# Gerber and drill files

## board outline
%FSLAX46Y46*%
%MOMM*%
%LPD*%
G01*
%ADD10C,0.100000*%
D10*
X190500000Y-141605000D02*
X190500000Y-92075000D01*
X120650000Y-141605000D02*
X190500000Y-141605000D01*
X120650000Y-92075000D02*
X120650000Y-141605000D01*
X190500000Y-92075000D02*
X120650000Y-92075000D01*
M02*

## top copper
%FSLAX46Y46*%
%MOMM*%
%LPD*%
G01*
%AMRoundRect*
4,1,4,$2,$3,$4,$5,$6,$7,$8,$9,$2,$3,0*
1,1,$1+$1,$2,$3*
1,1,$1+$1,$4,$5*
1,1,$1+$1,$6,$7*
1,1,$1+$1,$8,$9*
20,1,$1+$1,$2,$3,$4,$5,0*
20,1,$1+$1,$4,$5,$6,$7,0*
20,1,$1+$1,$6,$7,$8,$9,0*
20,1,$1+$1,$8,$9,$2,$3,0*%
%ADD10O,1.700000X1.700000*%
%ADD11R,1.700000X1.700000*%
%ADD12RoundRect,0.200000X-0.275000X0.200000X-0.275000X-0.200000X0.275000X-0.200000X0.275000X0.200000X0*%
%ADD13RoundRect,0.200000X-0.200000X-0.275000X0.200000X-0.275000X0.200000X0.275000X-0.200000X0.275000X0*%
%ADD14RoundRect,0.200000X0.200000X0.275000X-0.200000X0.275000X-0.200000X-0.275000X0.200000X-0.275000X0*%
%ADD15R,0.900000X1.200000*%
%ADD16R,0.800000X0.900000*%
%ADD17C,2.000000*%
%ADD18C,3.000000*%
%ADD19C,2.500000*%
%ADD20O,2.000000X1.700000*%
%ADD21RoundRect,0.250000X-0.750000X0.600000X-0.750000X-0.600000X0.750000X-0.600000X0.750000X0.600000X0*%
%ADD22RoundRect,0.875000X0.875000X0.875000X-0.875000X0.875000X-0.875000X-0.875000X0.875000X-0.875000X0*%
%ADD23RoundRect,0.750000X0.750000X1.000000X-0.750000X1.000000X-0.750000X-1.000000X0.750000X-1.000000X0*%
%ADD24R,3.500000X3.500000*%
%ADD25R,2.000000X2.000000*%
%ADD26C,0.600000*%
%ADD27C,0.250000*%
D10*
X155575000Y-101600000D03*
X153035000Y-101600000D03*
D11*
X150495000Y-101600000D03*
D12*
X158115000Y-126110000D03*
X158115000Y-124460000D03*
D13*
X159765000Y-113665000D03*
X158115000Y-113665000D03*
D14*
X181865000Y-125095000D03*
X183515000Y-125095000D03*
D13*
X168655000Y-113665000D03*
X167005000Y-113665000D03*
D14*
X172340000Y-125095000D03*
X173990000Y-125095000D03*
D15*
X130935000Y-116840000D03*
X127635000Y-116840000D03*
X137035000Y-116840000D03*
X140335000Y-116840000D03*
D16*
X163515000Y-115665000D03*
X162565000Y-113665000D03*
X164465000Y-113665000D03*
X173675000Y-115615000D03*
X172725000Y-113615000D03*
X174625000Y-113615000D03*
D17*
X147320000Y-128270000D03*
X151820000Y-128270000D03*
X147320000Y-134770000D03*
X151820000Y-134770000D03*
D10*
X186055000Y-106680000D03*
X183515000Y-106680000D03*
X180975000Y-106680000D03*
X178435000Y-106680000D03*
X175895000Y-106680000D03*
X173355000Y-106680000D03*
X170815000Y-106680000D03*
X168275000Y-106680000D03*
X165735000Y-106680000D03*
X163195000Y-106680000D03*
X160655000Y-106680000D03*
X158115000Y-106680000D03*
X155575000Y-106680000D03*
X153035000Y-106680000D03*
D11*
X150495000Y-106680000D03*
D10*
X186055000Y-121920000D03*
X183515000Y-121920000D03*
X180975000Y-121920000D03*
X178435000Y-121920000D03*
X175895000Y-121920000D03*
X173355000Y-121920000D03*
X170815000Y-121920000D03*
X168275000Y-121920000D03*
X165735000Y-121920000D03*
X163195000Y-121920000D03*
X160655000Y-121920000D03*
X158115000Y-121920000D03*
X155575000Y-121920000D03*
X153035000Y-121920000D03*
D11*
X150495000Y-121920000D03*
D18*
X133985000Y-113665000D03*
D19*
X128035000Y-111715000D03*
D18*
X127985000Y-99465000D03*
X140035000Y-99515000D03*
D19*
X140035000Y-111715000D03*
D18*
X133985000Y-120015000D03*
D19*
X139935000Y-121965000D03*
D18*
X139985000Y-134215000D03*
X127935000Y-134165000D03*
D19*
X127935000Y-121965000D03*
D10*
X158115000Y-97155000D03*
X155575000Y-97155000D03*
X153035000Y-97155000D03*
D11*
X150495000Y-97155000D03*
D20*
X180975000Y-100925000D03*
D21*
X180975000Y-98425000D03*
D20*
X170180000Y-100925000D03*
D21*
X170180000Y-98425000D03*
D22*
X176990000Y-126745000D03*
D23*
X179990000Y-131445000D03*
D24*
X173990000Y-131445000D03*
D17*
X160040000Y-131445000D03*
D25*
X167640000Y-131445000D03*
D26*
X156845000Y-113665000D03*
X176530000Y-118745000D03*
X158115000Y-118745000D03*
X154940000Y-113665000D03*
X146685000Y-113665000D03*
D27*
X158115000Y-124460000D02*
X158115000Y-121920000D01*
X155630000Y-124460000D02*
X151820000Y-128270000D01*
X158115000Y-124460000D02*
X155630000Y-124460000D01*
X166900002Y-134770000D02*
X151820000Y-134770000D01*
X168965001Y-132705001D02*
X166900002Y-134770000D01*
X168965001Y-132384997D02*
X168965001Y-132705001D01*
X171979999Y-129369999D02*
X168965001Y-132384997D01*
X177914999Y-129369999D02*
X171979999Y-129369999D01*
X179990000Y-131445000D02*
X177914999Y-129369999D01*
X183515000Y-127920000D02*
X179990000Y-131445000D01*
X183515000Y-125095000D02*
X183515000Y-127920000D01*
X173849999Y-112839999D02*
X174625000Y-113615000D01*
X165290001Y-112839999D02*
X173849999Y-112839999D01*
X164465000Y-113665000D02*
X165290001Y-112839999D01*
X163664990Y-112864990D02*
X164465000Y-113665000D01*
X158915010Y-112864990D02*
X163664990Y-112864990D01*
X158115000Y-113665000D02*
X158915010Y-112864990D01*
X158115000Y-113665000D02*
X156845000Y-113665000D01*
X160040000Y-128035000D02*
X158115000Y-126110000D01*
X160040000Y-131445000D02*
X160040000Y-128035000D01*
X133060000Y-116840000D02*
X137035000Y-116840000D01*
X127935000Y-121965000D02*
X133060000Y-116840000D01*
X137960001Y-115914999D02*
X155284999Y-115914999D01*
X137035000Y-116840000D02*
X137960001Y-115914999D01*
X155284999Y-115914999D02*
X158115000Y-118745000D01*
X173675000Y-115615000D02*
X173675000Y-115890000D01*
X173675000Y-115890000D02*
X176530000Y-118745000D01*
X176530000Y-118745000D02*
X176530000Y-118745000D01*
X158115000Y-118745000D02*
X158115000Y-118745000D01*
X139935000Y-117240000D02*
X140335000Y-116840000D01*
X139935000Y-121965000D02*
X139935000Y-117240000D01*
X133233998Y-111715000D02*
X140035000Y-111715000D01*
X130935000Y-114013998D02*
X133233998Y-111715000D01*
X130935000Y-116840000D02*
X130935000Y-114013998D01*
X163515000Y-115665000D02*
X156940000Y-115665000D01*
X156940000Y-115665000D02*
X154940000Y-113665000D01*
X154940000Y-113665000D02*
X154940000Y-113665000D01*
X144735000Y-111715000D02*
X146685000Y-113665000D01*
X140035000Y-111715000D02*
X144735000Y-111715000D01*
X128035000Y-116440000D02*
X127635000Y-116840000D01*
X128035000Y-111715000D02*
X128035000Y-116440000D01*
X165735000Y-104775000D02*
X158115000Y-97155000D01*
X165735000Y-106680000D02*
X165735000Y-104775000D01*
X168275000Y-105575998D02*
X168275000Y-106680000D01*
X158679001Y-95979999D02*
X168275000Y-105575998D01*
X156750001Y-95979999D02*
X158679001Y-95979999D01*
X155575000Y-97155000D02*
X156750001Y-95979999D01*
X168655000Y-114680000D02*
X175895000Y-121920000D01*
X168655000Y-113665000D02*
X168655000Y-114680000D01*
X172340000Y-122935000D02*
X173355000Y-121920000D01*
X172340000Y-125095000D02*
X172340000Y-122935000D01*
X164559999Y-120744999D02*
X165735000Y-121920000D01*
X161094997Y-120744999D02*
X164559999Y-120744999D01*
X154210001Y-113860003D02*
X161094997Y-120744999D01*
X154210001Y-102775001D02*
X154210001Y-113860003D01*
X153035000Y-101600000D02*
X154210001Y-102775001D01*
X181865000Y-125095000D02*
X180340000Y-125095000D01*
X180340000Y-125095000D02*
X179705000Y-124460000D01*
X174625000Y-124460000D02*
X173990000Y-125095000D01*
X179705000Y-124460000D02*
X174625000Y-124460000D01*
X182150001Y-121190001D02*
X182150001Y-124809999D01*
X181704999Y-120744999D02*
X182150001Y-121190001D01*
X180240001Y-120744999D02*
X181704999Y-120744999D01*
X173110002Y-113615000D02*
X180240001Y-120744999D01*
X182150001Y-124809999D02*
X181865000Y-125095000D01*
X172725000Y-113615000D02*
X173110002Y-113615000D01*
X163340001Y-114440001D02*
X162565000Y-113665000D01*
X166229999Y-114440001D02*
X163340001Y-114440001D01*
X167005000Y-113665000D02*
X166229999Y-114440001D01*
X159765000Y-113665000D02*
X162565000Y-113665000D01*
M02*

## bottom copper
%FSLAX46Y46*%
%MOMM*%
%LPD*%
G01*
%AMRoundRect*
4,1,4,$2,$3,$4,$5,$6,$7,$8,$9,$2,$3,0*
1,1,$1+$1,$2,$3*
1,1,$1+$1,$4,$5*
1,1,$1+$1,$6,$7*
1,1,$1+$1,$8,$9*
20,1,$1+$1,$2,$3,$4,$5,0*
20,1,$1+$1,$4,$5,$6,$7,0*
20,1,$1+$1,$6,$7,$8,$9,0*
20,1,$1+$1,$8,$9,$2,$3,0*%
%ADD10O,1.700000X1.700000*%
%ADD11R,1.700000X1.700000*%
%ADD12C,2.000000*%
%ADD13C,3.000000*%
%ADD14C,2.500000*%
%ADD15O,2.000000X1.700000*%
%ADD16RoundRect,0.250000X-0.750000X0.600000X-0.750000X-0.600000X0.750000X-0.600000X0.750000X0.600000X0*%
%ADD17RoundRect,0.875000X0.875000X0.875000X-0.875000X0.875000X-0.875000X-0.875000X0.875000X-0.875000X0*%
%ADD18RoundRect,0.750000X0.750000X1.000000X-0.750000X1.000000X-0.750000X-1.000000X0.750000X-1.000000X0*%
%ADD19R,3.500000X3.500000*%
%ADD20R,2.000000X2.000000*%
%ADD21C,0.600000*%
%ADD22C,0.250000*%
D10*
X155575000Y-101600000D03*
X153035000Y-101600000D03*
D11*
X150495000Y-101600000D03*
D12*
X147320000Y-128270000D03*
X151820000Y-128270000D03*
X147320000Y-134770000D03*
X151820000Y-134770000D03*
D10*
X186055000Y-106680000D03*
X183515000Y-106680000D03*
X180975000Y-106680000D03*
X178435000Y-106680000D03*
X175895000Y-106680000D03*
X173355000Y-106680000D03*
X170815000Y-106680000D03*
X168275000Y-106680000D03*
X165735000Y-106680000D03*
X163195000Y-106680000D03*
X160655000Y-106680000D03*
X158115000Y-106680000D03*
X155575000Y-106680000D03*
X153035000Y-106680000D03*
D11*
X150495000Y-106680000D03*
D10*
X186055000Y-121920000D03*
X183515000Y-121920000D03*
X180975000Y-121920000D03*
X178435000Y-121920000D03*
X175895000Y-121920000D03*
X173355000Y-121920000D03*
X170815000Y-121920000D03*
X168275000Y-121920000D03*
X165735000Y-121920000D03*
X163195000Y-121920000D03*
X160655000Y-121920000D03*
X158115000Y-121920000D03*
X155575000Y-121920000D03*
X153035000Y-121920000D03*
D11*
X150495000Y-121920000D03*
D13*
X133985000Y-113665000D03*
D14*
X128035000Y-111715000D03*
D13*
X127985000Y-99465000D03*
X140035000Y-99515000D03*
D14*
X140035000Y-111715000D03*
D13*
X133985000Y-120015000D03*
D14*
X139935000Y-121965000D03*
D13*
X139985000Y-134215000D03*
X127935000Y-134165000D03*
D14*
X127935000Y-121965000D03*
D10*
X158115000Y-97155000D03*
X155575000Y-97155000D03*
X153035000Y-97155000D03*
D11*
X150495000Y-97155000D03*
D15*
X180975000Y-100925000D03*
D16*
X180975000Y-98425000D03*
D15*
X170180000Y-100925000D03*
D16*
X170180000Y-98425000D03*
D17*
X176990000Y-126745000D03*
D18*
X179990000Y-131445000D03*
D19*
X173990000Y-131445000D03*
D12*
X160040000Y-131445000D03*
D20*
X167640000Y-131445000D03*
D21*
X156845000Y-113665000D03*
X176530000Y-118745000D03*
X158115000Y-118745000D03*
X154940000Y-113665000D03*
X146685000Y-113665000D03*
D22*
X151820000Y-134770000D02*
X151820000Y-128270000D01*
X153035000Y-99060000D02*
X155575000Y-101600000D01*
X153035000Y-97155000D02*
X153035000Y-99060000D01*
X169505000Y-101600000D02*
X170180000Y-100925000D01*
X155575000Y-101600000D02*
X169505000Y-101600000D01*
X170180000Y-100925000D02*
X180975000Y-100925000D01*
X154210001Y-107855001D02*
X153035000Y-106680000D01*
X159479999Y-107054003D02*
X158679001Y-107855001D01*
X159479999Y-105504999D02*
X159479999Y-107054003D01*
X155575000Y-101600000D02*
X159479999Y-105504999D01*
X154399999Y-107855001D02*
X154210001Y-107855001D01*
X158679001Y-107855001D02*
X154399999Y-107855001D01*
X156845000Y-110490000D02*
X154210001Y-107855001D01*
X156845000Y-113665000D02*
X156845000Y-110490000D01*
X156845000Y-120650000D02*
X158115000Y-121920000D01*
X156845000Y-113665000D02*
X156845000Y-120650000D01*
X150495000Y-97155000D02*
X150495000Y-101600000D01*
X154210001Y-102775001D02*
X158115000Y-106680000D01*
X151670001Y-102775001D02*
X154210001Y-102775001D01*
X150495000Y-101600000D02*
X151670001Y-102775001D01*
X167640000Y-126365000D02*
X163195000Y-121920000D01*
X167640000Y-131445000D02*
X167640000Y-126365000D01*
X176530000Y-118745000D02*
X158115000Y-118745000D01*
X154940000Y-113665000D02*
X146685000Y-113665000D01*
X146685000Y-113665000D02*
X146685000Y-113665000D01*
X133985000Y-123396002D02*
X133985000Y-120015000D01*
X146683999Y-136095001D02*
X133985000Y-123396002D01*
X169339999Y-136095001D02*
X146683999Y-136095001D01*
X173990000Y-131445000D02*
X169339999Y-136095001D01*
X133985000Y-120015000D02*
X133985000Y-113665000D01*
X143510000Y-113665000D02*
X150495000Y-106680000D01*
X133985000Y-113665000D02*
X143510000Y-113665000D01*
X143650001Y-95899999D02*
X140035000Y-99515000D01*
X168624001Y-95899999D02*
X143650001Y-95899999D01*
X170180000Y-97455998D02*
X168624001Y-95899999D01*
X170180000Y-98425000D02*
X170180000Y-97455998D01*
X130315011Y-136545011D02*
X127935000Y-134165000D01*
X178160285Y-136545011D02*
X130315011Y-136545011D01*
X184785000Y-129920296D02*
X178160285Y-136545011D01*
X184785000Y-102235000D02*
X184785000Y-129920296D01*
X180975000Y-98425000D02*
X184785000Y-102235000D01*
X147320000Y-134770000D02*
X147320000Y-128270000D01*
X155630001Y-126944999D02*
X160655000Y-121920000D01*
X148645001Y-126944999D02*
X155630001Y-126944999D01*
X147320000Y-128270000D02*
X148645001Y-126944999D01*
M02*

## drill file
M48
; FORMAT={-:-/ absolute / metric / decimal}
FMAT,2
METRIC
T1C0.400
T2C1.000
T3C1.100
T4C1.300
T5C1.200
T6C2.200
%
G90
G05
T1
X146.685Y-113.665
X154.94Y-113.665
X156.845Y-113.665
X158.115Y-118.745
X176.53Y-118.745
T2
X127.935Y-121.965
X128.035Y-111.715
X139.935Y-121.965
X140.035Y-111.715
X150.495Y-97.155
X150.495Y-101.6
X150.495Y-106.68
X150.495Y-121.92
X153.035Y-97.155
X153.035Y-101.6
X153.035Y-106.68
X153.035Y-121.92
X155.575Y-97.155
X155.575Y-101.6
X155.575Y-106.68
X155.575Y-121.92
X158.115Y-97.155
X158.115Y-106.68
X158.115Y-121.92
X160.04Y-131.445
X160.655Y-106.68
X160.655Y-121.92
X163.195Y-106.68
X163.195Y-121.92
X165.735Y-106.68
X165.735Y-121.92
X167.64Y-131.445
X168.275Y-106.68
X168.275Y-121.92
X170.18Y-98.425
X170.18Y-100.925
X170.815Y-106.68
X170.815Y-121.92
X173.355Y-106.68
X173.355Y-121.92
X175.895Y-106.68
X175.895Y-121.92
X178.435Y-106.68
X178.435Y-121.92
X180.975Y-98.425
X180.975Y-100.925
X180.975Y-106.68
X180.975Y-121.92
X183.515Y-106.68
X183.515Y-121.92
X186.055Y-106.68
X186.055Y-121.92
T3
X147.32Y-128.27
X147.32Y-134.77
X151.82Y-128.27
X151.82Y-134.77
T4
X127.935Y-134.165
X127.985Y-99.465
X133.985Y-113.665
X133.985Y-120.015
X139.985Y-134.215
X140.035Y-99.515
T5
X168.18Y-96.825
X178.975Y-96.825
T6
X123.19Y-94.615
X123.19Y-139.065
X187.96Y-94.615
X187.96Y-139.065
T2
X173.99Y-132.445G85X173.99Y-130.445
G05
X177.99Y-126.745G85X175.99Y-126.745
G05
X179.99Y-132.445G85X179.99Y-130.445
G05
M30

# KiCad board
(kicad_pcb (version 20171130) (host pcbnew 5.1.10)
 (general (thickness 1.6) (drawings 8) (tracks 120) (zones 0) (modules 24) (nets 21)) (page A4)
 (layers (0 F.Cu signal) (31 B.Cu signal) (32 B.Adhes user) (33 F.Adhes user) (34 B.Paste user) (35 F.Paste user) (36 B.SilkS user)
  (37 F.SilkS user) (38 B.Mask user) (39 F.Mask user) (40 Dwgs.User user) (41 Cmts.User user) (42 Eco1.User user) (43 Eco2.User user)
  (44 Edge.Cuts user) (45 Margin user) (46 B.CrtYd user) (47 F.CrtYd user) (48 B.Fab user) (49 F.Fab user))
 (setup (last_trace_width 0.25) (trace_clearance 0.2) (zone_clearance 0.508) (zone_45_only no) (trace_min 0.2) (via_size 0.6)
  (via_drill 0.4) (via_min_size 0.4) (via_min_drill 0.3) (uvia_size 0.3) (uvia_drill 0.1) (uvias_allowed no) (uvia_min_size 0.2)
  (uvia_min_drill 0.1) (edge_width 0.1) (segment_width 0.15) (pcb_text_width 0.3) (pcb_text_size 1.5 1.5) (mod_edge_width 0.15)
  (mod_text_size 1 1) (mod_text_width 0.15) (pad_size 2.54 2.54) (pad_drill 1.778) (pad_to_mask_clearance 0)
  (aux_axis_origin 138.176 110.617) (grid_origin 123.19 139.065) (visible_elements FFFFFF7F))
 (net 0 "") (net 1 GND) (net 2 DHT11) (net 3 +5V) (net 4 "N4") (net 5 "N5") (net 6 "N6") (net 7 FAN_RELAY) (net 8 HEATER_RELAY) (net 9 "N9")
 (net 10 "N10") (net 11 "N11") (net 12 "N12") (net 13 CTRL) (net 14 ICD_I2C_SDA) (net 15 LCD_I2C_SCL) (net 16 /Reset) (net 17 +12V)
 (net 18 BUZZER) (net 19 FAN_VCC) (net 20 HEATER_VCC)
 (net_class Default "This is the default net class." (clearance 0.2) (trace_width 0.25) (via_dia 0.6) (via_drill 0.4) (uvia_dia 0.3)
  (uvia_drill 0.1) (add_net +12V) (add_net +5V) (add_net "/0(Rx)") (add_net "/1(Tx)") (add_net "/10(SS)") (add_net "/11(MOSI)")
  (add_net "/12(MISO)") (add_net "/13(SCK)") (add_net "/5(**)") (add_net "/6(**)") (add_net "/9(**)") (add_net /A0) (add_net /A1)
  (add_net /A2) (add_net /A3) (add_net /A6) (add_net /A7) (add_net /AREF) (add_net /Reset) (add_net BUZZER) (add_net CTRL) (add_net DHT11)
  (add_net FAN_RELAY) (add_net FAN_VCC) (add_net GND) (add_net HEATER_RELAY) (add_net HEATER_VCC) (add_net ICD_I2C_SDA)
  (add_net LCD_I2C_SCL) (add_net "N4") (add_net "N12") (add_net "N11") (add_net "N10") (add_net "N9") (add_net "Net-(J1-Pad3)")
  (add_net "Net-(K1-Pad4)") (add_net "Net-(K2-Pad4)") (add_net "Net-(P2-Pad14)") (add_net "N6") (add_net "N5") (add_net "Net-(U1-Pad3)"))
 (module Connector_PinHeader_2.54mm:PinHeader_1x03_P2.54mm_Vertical (layer F.Cu) (at 150.495 101.6 90)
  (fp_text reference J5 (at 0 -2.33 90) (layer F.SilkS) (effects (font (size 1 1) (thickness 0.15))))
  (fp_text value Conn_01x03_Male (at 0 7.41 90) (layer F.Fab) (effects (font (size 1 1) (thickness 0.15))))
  (pad 3 thru_hole oval (at 0 5.08 90) (size 1.7 1.7) (drill 1) (layers *.Cu *.Mask) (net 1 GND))
  (pad 2 thru_hole oval (at 0 2.54 90) (size 1.7 1.7) (drill 1) (layers *.Cu *.Mask) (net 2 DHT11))
  (pad 1 thru_hole rect (at 0 0 90) (size 1.7 1.7) (drill 1) (layers *.Cu *.Mask) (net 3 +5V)))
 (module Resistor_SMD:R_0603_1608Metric (layer F.Cu) (at 158.115 125.285 270)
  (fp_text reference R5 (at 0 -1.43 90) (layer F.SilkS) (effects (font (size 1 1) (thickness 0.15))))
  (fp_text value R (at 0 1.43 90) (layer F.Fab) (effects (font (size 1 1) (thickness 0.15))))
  (pad 2 smd roundrect (at 0.825 0 270) (size 0.8 0.95) (layers F.Cu F.Paste F.Mask) (roundrect_rratio 0.25) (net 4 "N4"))
  (pad 1 smd roundrect (at -0.825 0 270) (size 0.8 0.95) (layers F.Cu F.Paste F.Mask) (roundrect_rratio 0.25) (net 1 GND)))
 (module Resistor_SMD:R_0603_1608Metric (layer F.Cu) (at 158.94 113.665)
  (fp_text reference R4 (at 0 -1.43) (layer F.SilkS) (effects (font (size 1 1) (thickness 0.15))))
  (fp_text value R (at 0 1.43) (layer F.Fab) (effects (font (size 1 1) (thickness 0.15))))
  (pad 2 smd roundrect (at 0.825 0) (size 0.8 0.95) (layers F.Cu F.Paste F.Mask) (roundrect_rratio 0.25) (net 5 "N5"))
  (pad 1 smd roundrect (at -0.825 0) (size 0.8 0.95) (layers F.Cu F.Paste F.Mask) (roundrect_rratio 0.25) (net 1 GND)))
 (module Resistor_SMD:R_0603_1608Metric (layer F.Cu) (at 182.69 125.095 180)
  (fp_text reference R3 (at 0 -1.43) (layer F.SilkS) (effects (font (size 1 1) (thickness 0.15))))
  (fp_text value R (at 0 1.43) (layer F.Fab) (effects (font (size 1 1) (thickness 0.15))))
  (pad 2 smd roundrect (at 0.825 0 180) (size 0.8 0.95) (layers F.Cu F.Paste F.Mask) (roundrect_rratio 0.25) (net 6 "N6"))
  (pad 1 smd roundrect (at -0.825 0 180) (size 0.8 0.95) (layers F.Cu F.Paste F.Mask) (roundrect_rratio 0.25) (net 1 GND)))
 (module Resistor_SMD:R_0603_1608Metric (layer F.Cu) (at 167.83 113.665)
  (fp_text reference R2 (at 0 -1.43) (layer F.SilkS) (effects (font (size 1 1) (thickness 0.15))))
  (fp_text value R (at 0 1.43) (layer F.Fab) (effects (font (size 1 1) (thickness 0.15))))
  (pad 2 smd roundrect (at 0.825 0) (size 0.8 0.95) (layers F.Cu F.Paste F.Mask) (roundrect_rratio 0.25) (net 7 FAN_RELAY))
  (pad 1 smd roundrect (at -0.825 0) (size 0.8 0.95) (layers F.Cu F.Paste F.Mask) (roundrect_rratio 0.25) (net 5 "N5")))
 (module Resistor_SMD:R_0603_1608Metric (layer F.Cu) (at 173.165 125.095 180)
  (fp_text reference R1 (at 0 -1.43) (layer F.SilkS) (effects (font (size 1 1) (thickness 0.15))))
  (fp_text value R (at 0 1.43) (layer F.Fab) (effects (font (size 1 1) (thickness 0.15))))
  (pad 2 smd roundrect (at 0.825 0 180) (size 0.8 0.95) (layers F.Cu F.Paste F.Mask) (roundrect_rratio 0.25) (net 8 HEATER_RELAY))
  (pad 1 smd roundrect (at -0.825 0 180) (size 0.8 0.95) (layers F.Cu F.Paste F.Mask) (roundrect_rratio 0.25) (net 6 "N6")))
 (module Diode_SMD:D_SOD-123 (layer F.Cu) (at 129.285 116.84)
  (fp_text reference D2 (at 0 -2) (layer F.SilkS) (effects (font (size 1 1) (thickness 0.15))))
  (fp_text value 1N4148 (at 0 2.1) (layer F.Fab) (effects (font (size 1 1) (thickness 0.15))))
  (pad 2 smd rect (at 1.65 0) (size 0.9 1.2) (layers F.Cu F.Paste F.Mask) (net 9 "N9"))
  (pad 1 smd rect (at -1.65 0) (size 0.9 1.2) (layers F.Cu F.Paste F.Mask) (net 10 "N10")))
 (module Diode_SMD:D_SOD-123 (layer F.Cu) (at 138.685 116.84 180)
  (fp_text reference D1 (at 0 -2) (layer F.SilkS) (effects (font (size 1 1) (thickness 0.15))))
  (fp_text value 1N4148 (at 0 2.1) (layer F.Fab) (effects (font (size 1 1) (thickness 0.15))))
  (pad 2 smd rect (at 1.65 0 180) (size 0.9 1.2) (layers F.Cu F.Paste F.Mask) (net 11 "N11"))
  (pad 1 smd rect (at -1.65 0 180) (size 0.9 1.2) (layers F.Cu F.Paste F.Mask) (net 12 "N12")))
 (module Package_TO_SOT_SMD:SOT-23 (layer F.Cu) (at 163.515 114.665 270)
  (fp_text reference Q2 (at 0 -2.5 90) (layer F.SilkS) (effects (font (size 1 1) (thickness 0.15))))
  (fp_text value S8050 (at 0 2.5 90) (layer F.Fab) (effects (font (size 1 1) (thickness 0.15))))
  (pad 3 smd rect (at 1 0 270) (size 0.9 0.8) (layers F.Cu F.Paste F.Mask) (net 9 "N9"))
  (pad 2 smd rect (at -1 0.95 270) (size 0.9 0.8) (layers F.Cu F.Paste F.Mask) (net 5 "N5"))
  (pad 1 smd rect (at -1 -0.95 270) (size 0.9 0.8) (layers F.Cu F.Paste F.Mask) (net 1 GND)))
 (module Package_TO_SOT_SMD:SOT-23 (layer F.Cu) (at 173.675 114.615 270)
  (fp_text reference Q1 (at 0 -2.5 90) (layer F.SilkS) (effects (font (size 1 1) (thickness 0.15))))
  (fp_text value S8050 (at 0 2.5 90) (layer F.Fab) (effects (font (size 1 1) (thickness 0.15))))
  (pad 3 smd rect (at 1 0 270) (size 0.9 0.8) (layers F.Cu F.Paste F.Mask) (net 11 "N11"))
  (pad 2 smd rect (at -1 0.95 270) (size 0.9 0.8) (layers F.Cu F.Paste F.Mask) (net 6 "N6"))
  (pad 1 smd rect (at -1 -0.95 270) (size 0.9 0.8) (layers F.Cu F.Paste F.Mask) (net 1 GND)))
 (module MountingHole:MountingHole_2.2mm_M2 (layer F.Cu) (at 187.96 94.615)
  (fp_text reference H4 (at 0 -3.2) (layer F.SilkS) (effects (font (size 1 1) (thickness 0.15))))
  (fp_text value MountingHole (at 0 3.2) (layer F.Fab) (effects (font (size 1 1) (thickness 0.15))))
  (pad 1 np_thru_hole circle (at 0 0) (size 2.2 2.2) (drill 2.2) (layers *.Cu *.Mask)))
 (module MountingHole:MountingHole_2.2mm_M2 (layer F.Cu) (at 187.96 139.065)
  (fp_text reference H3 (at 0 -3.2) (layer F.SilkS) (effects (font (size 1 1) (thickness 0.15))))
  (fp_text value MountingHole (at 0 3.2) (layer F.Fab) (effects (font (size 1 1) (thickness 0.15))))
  (pad 1 np_thru_hole circle (at 0 0) (size 2.2 2.2) (drill 2.2) (layers *.Cu *.Mask)))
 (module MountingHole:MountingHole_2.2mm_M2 (layer F.Cu) (at 123.19 139.065)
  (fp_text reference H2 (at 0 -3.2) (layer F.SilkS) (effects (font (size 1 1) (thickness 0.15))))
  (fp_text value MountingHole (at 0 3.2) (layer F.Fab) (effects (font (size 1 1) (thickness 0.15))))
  (pad 1 np_thru_hole circle (at 0 0) (size 2.2 2.2) (drill 2.2) (layers *.Cu *.Mask)))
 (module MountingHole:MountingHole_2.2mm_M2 (layer F.Cu) (at 123.19 94.615)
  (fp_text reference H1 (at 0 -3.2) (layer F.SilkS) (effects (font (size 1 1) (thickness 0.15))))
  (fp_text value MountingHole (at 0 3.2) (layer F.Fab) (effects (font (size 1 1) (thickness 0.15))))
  (pad 1 np_thru_hole circle (at 0 0) (size 2.2 2.2) (drill 2.2) (layers *.Cu *.Mask)))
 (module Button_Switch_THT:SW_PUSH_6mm (layer F.Cu) (at 147.32 134.77 90)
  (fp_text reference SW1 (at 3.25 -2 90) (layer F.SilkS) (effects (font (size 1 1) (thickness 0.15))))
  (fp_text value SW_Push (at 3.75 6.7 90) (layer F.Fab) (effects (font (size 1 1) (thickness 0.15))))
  (pad 1 thru_hole circle (at 6.5 0 180) (size 2 2) (drill 1.1) (layers *.Cu *.Mask) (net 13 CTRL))
  (pad 2 thru_hole circle (at 6.5 4.5 180) (size 2 2) (drill 1.1) (layers *.Cu *.Mask) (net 1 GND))
  (pad 1 thru_hole circle (at 0 0 180) (size 2 2) (drill 1.1) (layers *.Cu *.Mask) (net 13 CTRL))
  (pad 2 thru_hole circle (at 0 4.5 180) (size 2 2) (drill 1.1) (layers *.Cu *.Mask) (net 1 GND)))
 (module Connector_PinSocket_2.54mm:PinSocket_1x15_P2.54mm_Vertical (layer F.Cu) (at 150.495 106.68 90)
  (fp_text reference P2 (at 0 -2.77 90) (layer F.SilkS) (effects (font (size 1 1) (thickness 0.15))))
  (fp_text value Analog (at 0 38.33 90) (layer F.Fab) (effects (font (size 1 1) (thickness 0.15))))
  (pad 15 thru_hole oval (at 0 35.56 90) (size 1.7 1.7) (drill 1) (layers *.Cu *.Mask))
  (pad 14 thru_hole oval (at 0 33.02 90) (size 1.7 1.7) (drill 1) (layers *.Cu *.Mask))
  (pad 13 thru_hole oval (at 0 30.48 90) (size 1.7 1.7) (drill 1) (layers *.Cu *.Mask))
  (pad 12 thru_hole oval (at 0 27.94 90) (size 1.7 1.7) (drill 1) (layers *.Cu *.Mask))
  (pad 11 thru_hole oval (at 0 25.4 90) (size 1.7 1.7) (drill 1) (layers *.Cu *.Mask))
  (pad 10 thru_hole oval (at 0 22.86 90) (size 1.7 1.7) (drill 1) (layers *.Cu *.Mask))
  (pad 9 thru_hole oval (at 0 20.32 90) (size 1.7 1.7) (drill 1) (layers *.Cu *.Mask))
  (pad 8 thru_hole oval (at 0 17.78 90) (size 1.7 1.7) (drill 1) (layers *.Cu *.Mask) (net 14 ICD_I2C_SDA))
  (pad 7 thru_hole oval (at 0 15.24 90) (size 1.7 1.7) (drill 1) (layers *.Cu *.Mask) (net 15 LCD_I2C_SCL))
  (pad 6 thru_hole oval (at 0 12.7 90) (size 1.7 1.7) (drill 1) (layers *.Cu *.Mask))
  (pad 5 thru_hole oval (at 0 10.16 90) (size 1.7 1.7) (drill 1) (layers *.Cu *.Mask))
  (pad 4 thru_hole oval (at 0 7.62 90) (size 1.7 1.7) (drill 1) (layers *.Cu *.Mask) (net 3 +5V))
  (pad 3 thru_hole oval (at 0 5.08 90) (size 1.7 1.7) (drill 1) (layers *.Cu *.Mask) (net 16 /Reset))
  (pad 2 thru_hole oval (at 0 2.54 90) (size 1.7 1.7) (drill 1) (layers *.Cu *.Mask) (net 1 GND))
  (pad 1 thru_hole rect (at 0 0 90) (size 1.7 1.7) (drill 1) (layers *.Cu *.Mask) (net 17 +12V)))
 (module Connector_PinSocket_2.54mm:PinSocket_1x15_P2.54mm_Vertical (layer F.Cu) (at 150.495 121.92 90)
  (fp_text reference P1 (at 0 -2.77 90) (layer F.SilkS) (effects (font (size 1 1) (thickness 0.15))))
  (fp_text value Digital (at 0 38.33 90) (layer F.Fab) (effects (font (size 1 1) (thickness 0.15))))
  (pad 15 thru_hole oval (at 0 35.56 90) (size 1.7 1.7) (drill 1) (layers *.Cu *.Mask))
  (pad 14 thru_hole oval (at 0 33.02 90) (size 1.7 1.7) (drill 1) (layers *.Cu *.Mask))
  (pad 13 thru_hole oval (at 0 30.48 90) (size 1.7 1.7) (drill 1) (layers *.Cu *.Mask))
  (pad 12 thru_hole oval (at 0 27.94 90) (size 1.7 1.7) (drill 1) (layers *.Cu *.Mask))
  (pad 11 thru_hole oval (at 0 25.4 90) (size 1.7 1.7) (drill 1) (layers *.Cu *.Mask) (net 7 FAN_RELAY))
  (pad 10 thru_hole oval (at 0 22.86 90) (size 1.7 1.7) (drill 1) (layers *.Cu *.Mask) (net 8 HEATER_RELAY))
  (pad 9 thru_hole oval (at 0 20.32 90) (size 1.7 1.7) (drill 1) (layers *.Cu *.Mask))
  (pad 8 thru_hole oval (at 0 17.78 90) (size 1.7 1.7) (drill 1) (layers *.Cu *.Mask))
  (pad 7 thru_hole oval (at 0 15.24 90) (size 1.7 1.7) (drill 1) (layers *.Cu *.Mask) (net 2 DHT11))
  (pad 6 thru_hole oval (at 0 12.7 90) (size 1.7 1.7) (drill 1) (layers *.Cu *.Mask) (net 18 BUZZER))
  (pad 5 thru_hole oval (at 0 10.16 90) (size 1.7 1.7) (drill 1) (layers *.Cu *.Mask) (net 13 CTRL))
  (pad 4 thru_hole oval (at 0 7.62 90) (size 1.7 1.7) (drill 1) (layers *.Cu *.Mask) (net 1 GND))
  (pad 3 thru_hole oval (at 0 5.08 90) (size 1.7 1.7) (drill 1) (layers *.Cu *.Mask) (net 16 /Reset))
  (pad 2 thru_hole oval (at 0 2.54 90) (size 1.7 1.7) (drill 1) (layers *.Cu *.Mask))
  (pad 1 thru_hole rect (at 0 0 90) (size 1.7 1.7) (drill 1) (layers *.Cu *.Mask)))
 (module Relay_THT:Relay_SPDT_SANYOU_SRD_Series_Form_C (layer F.Cu) (at 133.985 113.665 90)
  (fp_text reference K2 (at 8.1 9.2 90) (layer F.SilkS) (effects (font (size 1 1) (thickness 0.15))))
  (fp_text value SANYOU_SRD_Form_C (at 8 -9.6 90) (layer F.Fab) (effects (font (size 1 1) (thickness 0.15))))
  (pad 1 thru_hole circle (at 0 0 180) (size 3 3) (drill 1.3) (layers *.Cu *.Mask) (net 17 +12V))
  (pad 5 thru_hole circle (at 1.95 -5.95 180) (size 2.5 2.5) (drill 1) (layers *.Cu *.Mask) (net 10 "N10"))
  (pad 4 thru_hole circle (at 14.2 -6 180) (size 3 3) (drill 1.3) (layers *.Cu *.Mask))
  (pad 3 thru_hole circle (at 14.15 6.05 180) (size 3 3) (drill 1.3) (layers *.Cu *.Mask) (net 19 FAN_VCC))
  (pad 2 thru_hole circle (at 1.95 6.05 180) (size 2.5 2.5) (drill 1) (layers *.Cu *.Mask) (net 9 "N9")))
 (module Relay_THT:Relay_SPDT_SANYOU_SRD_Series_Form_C (layer F.Cu) (at 133.985 120.015 270)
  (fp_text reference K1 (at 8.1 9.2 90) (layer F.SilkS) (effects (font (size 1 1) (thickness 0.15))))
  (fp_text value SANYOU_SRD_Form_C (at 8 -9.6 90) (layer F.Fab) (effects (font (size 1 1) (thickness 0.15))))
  (pad 1 thru_hole circle (at 0 0) (size 3 3) (drill 1.3) (layers *.Cu *.Mask) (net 17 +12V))
  (pad 5 thru_hole circle (at 1.95 -5.95) (size 2.5 2.5) (drill 1) (layers *.Cu *.Mask) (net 12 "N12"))
  (pad 4 thru_hole circle (at 14.2 -6) (size 3 3) (drill 1.3) (layers *.Cu *.Mask))
  (pad 3 thru_hole circle (at 14.15 6.05) (size 3 3) (drill 1.3) (layers *.Cu *.Mask) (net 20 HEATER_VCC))
  (pad 2 thru_hole circle (at 1.95 6.05) (size 2.5 2.5) (drill 1) (layers *.Cu *.Mask) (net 11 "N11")))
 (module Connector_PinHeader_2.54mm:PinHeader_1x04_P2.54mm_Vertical (layer F.Cu) (at 150.495 97.155 90)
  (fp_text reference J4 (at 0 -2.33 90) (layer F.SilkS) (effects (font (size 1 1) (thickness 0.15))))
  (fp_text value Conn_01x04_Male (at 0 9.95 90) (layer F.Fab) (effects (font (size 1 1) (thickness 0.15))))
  (pad 4 thru_hole oval (at 0 7.62 90) (size 1.7 1.7) (drill 1) (layers *.Cu *.Mask) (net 15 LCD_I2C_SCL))
  (pad 3 thru_hole oval (at 0 5.08 90) (size 1.7 1.7) (drill 1) (layers *.Cu *.Mask) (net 14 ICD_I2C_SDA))
  (pad 2 thru_hole oval (at 0 2.54 90) (size 1.7 1.7) (drill 1) (layers *.Cu *.Mask) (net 1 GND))
  (pad 1 thru_hole rect (at 0 0 90) (size 1.7 1.7) (drill 1) (layers *.Cu *.Mask) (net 3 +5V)))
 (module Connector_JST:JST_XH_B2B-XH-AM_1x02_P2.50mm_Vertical (layer F.Cu) (at 180.975 98.425 270)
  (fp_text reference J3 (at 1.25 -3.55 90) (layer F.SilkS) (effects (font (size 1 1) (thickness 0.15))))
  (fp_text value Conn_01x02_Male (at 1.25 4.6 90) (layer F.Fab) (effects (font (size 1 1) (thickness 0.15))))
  (pad "" np_thru_hole circle (at -1.6 2 270) (size 1.2 1.2) (drill 1.2) (layers *.Cu *.Mask))
  (pad 2 thru_hole oval (at 2.5 0 270) (size 1.7 2) (drill 1) (layers *.Cu *.Mask) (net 1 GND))
  (pad 1 thru_hole roundrect (at 0 0 270) (size 1.7 2) (drill 1) (layers *.Cu *.Mask) (roundrect_rratio 0.147059) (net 20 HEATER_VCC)))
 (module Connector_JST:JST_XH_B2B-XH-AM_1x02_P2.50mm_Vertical (layer F.Cu) (at 170.18 98.425 270)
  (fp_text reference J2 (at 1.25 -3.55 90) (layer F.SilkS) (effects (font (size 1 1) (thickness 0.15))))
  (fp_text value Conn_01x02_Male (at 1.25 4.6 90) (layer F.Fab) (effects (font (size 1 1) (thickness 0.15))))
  (pad "" np_thru_hole circle (at -1.6 2 270) (size 1.2 1.2) (drill 1.2) (layers *.Cu *.Mask))
  (pad 2 thru_hole oval (at 2.5 0 270) (size 1.7 2) (drill 1) (layers *.Cu *.Mask) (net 1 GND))
  (pad 1 thru_hole roundrect (at 0 0 270) (size 1.7 2) (drill 1) (layers *.Cu *.Mask) (roundrect_rratio 0.147059) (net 19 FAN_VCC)))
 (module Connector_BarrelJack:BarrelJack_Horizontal (layer F.Cu) (at 173.99 131.445 180)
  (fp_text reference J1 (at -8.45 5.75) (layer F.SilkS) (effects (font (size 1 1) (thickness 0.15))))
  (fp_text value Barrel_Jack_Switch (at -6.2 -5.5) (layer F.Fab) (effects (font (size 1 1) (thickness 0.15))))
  (pad 3 thru_hole roundrect (at -3 4.7 180) (size 3.5 3.5) (drill oval 3 1) (layers *.Cu *.Mask) (roundrect_rratio 0.25))
  (pad 2 thru_hole roundrect (at -6 0 180) (size 3 3.5) (drill oval 1 3) (layers *.Cu *.Mask) (roundrect_rratio 0.25) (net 1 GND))
  (pad 1 thru_hole rect (at 0 0 180) (size 3.5 3.5) (drill oval 1 3) (layers *.Cu *.Mask) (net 17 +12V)))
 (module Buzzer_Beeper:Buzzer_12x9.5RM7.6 (layer F.Cu) (at 167.64 131.445 180)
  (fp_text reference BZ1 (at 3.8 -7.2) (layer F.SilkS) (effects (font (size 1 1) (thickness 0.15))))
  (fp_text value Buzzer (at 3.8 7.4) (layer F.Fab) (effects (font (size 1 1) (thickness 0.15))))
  (pad 2 thru_hole circle (at 7.6 0 180) (size 2 2) (drill 1) (layers *.Cu *.Mask) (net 4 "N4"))
  (pad 1 thru_hole rect (at 0 0 180) (size 2 2) (drill 1) (layers *.Cu *.Mask) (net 18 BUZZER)))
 (gr_line (start 190.5 141.605) (end 190.5 92.075) (angle 90) (layer Edge.Cuts) (width 0.1))
 (gr_line (start 120.65 141.605) (end 190.5 141.605) (angle 90) (layer Edge.Cuts) (width 0.1))
 (gr_line (start 120.65 92.075) (end 120.65 141.605) (angle 90) (layer Edge.Cuts) (width 0.1))
 (gr_line (start 190.5 92.075) (end 120.65 92.075) (angle 90) (layer Edge.Cuts) (width 0.1))
 (via (at 156.845 113.665) (size 0.6) (drill 0.4) (layers F.Cu B.Cu) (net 1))
 (segment (start 151.82 134.77) (end 151.82 128.27) (width 0.25) (layer B.Cu) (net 1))
 (segment (start 158.115 124.46) (end 158.115 121.92) (width 0.25) (layer F.Cu) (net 1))
 (segment (start 155.63 124.46) (end 151.82 128.27) (width 0.25) (layer F.Cu) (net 1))
 (segment (start 158.115 124.46) (end 155.63 124.46) (width 0.25) (layer F.Cu) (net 1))
 (segment (start 166.900002 134.77) (end 151.82 134.77) (width 0.25) (layer F.Cu) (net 1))
 (segment (start 168.965001 132.705001) (end 166.900002 134.77) (width 0.25) (layer F.Cu) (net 1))
 (segment (start 168.965001 132.384997) (end 168.965001 132.705001) (width 0.25) (layer F.Cu) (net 1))
 (segment (start 171.979999 129.369999) (end 168.965001 132.384997) (width 0.25) (layer F.Cu) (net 1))
 (segment (start 177.914999 129.369999) (end 171.979999 129.369999) (width 0.25) (layer F.Cu) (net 1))
 (segment (start 179.99 131.445) (end 177.914999 129.369999) (width 0.25) (layer F.Cu) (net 1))
 (segment (start 183.515 127.92) (end 179.99 131.445) (width 0.25) (layer F.Cu) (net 1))
 (segment (start 183.515 125.095) (end 183.515 127.92) (width 0.25) (layer F.Cu) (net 1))
 (segment (start 173.849999 112.839999) (end 174.625 113.615) (width 0.25) (layer F.Cu) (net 1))
 (segment (start 165.290001 112.839999) (end 173.849999 112.839999) (width 0.25) (layer F.Cu) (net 1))
 (segment (start 164.465 113.665) (end 165.290001 112.839999) (width 0.25) (layer F.Cu) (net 1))
 (segment (start 163.66499 112.86499) (end 164.465 113.665) (width 0.25) (layer F.Cu) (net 1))
 (segment (start 158.91501 112.86499) (end 163.66499 112.86499) (width 0.25) (layer F.Cu) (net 1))
 (segment (start 158.115 113.665) (end 158.91501 112.86499) (width 0.25) (layer F.Cu) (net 1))
 (segment (start 153.035 99.06) (end 155.575 101.6) (width 0.25) (layer B.Cu) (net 1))
 (segment (start 153.035 97.155) (end 153.035 99.06) (width 0.25) (layer B.Cu) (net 1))
 (segment (start 169.505 101.6) (end 170.18 100.925) (width 0.25) (layer B.Cu) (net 1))
 (segment (start 155.575 101.6) (end 169.505 101.6) (width 0.25) (layer B.Cu) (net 1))
 (segment (start 170.18 100.925) (end 180.975 100.925) (width 0.25) (layer B.Cu) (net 1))
 (segment (start 154.210001 107.855001) (end 153.035 106.68) (width 0.25) (layer B.Cu) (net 1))
 (segment (start 159.479999 107.054003) (end 158.679001 107.855001) (width 0.25) (layer B.Cu) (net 1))
 (segment (start 159.479999 105.504999) (end 159.479999 107.054003) (width 0.25) (layer B.Cu) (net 1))
 (segment (start 155.575 101.6) (end 159.479999 105.504999) (width 0.25) (layer B.Cu) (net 1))
 (segment (start 154.399999 107.855001) (end 154.210001 107.855001) (width 0.25) (layer B.Cu) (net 1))
 (segment (start 158.679001 107.855001) (end 154.399999 107.855001) (width 0.25) (layer B.Cu) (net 1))
 (segment (start 156.845 110.49) (end 154.210001 107.855001) (width 0.25) (layer B.Cu) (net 1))
 (segment (start 156.845 113.665) (end 156.845 110.49) (width 0.25) (layer B.Cu) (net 1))
 (segment (start 156.845 120.65) (end 158.115 121.92) (width 0.25) (layer B.Cu) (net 1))
 (segment (start 156.845 113.665) (end 156.845 120.65) (width 0.25) (layer B.Cu) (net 1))
 (segment (start 158.115 113.665) (end 156.845 113.665) (width 0.25) (layer F.Cu) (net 1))
 (segment (start 150.495 97.155) (end 150.495 101.6) (width 0.25) (layer B.Cu) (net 3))
 (segment (start 154.210001 102.775001) (end 158.115 106.68) (width 0.25) (layer B.Cu) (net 3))
 (segment (start 151.670001 102.775001) (end 154.210001 102.775001) (width 0.25) (layer B.Cu) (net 3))
 (segment (start 150.495 101.6) (end 151.670001 102.775001) (width 0.25) (layer B.Cu) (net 3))
 (segment (start 160.04 128.035) (end 158.115 126.11) (width 0.25) (layer F.Cu) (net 4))
 (segment (start 160.04 131.445) (end 160.04 128.035) (width 0.25) (layer F.Cu) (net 4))
 (segment (start 167.64 126.365) (end 163.195 121.92) (width 0.25) (layer B.Cu) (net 18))
 (segment (start 167.64 131.445) (end 167.64 126.365) (width 0.25) (layer B.Cu) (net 18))
 (segment (start 133.06 116.84) (end 137.035 116.84) (width 0.25) (layer F.Cu) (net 11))
 (segment (start 127.935 121.965) (end 133.06 116.84) (width 0.25) (layer F.Cu) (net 11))
 (segment (start 137.960001 115.914999) (end 155.284999 115.914999) (width 0.25) (layer F.Cu) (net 11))
 (segment (start 137.035 116.84) (end 137.960001 115.914999) (width 0.25) (layer F.Cu) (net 11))
 (segment (start 155.284999 115.914999) (end 158.115 118.745) (width 0.25) (layer F.Cu) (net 11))
 (segment (start 173.675 115.615) (end 173.675 115.89) (width 0.25) (layer F.Cu) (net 11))
 (segment (start 173.675 115.89) (end 176.53 118.745) (width 0.25) (layer F.Cu) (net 11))
 (segment (start 176.53 118.745) (end 176.53 118.745) (width 0.25) (layer F.Cu) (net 11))
 (via (at 176.53 118.745) (size 0.6) (drill 0.4) (layers F.Cu B.Cu) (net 11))
 (segment (start 158.115 118.745) (end 158.115 118.745) (width 0.25) (layer F.Cu) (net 11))
 (via (at 158.115 118.745) (size 0.6) (drill 0.4) (layers F.Cu B.Cu) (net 11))
 (segment (start 176.53 118.745) (end 158.115 118.745) (width 0.25) (layer B.Cu) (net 11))
 (segment (start 139.935 117.24) (end 140.335 116.84) (width 0.25) (layer F.Cu) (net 12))
 (segment (start 139.935 121.965) (end 139.935 117.24) (width 0.25) (layer F.Cu) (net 12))
 (segment (start 133.233998 111.715) (end 140.035 111.715) (width 0.25) (layer F.Cu) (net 9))
 (segment (start 130.935 114.013998) (end 133.233998 111.715) (width 0.25) (layer F.Cu) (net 9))
 (segment (start 130.935 116.84) (end 130.935 114.013998) (width 0.25) (layer F.Cu) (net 9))
 (segment (start 163.515 115.665) (end 156.94 115.665) (width 0.25) (layer F.Cu) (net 9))
 (segment (start 156.94 115.665) (end 154.94 113.665) (width 0.25) (layer F.Cu) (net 9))
 (segment (start 154.94 113.665) (end 154.94 113.665) (width 0.25) (layer F.Cu) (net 9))
 (via (at 154.94 113.665) (size 0.6) (drill 0.4) (layers F.Cu B.Cu) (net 9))
 (segment (start 154.94 113.665) (end 146.685 113.665) (width 0.25) (layer B.Cu) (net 9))
 (segment (start 146.685 113.665) (end 146.685 113.665) (width 0.25) (layer B.Cu) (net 9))
 (via (at 146.685 113.665) (size 0.6) (drill 0.4) (layers F.Cu B.Cu) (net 9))
 (segment (start 144.735 111.715) (end 146.685 113.665) (width 0.25) (layer F.Cu) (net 9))
 (segment (start 140.035 111.715) (end 144.735 111.715) (width 0.25) (layer F.Cu) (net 9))
 (segment (start 128.035 116.44) (end 127.635 116.84) (width 0.25) (layer F.Cu) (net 10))
 (segment (start 128.035 111.715) (end 128.035 116.44) (width 0.25) (layer F.Cu) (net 10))
 (segment (start 133.985 123.396002) (end 133.985 120.015) (width 0.25) (layer B.Cu) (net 17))
 (segment (start 146.683999 136.095001) (end 133.985 123.396002) (width 0.25) (layer B.Cu) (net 17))
 (segment (start 169.339999 136.095001) (end 146.683999 136.095001) (width 0.25) (layer B.Cu) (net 17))
 (segment (start 173.99 131.445) (end 169.339999 136.095001) (width 0.25) (layer B.Cu) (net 17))
 (segment (start 133.985 120.015) (end 133.985 113.665) (width 0.25) (layer B.Cu) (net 17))
 (segment (start 143.51 113.665) (end 150.495 106.68) (width 0.25) (layer B.Cu) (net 17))
 (segment (start 133.985 113.665) (end 143.51 113.665) (width 0.25) (layer B.Cu) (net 17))
 (segment (start 143.650001 95.899999) (end 140.035 99.515) (width 0.25) (layer B.Cu) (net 19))
 (segment (start 168.624001 95.899999) (end 143.650001 95.899999) (width 0.25) (layer B.Cu) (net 19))
 (segment (start 170.18 97.455998) (end 168.624001 95.899999) (width 0.25) (layer B.Cu) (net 19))
 (segment (start 170.18 98.425) (end 170.18 97.455998) (width 0.25) (layer B.Cu) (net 19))
 (segment (start 130.315011 136.545011) (end 127.935 134.165) (width 0.25) (layer B.Cu) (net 20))
 (segment (start 178.160285 136.545011) (end 130.315011 136.545011) (width 0.25) (layer B.Cu) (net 20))
 (segment (start 184.785 129.920296) (end 178.160285 136.545011) (width 0.25) (layer B.Cu) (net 20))
 (segment (start 184.785 102.235) (end 184.785 129.920296) (width 0.25) (layer B.Cu) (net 20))
 (segment (start 180.975 98.425) (end 184.785 102.235) (width 0.25) (layer B.Cu) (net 20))
 (segment (start 165.735 104.775) (end 158.115 97.155) (width 0.25) (layer F.Cu) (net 15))
 (segment (start 165.735 106.68) (end 165.735 104.775) (width 0.25) (layer F.Cu) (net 15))
 (segment (start 168.275 105.575998) (end 168.275 106.68) (width 0.25) (layer F.Cu) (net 14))
 (segment (start 158.679001 95.979999) (end 168.275 105.575998) (width 0.25) (layer F.Cu) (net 14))
 (segment (start 156.750001 95.979999) (end 158.679001 95.979999) (width 0.25) (layer F.Cu) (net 14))
 (segment (start 155.575 97.155) (end 156.750001 95.979999) (width 0.25) (layer F.Cu) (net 14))
 (segment (start 168.655 114.68) (end 175.895 121.92) (width 0.25) (layer F.Cu) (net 7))
 (segment (start 168.655 113.665) (end 168.655 114.68) (width 0.25) (layer F.Cu) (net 7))
 (segment (start 172.34 122.935) (end 173.355 121.92) (width 0.25) (layer F.Cu) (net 8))
 (segment (start 172.34 125.095) (end 172.34 122.935) (width 0.25) (layer F.Cu) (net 8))
 (segment (start 164.559999 120.744999) (end 165.735 121.92) (width 0.25) (layer F.Cu) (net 2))
 (segment (start 161.094997 120.744999) (end 164.559999 120.744999) (width 0.25) (layer F.Cu) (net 2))
 (segment (start 154.210001 113.860003) (end 161.094997 120.744999) (width 0.25) (layer F.Cu) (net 2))
 (segment (start 154.210001 102.775001) (end 154.210001 113.860003) (width 0.25) (layer F.Cu) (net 2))
 (segment (start 153.035 101.6) (end 154.210001 102.775001) (width 0.25) (layer F.Cu) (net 2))
 (segment (start 147.32 134.77) (end 147.32 128.27) (width 0.25) (layer B.Cu) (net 13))
 (segment (start 155.630001 126.944999) (end 160.655 121.92) (width 0.25) (layer B.Cu) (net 13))
 (segment (start 148.645001 126.944999) (end 155.630001 126.944999) (width 0.25) (layer B.Cu) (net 13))
 (segment (start 147.32 128.27) (end 148.645001 126.944999) (width 0.25) (layer B.Cu) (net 13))
 (segment (start 181.865 125.095) (end 180.34 125.095) (width 0.25) (layer F.Cu) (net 6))
 (segment (start 180.34 125.095) (end 179.705 124.46) (width 0.25) (layer F.Cu) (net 6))
 (segment (start 174.625 124.46) (end 173.99 125.095) (width 0.25) (layer F.Cu) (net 6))
 (segment (start 179.705 124.46) (end 174.625 124.46) (width 0.25) (layer F.Cu) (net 6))
 (segment (start 182.150001 121.190001) (end 182.150001 124.809999) (width 0.25) (layer F.Cu) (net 6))
 (segment (start 181.704999 120.744999) (end 182.150001 121.190001) (width 0.25) (layer F.Cu) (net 6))
 (segment (start 180.240001 120.744999) (end 181.704999 120.744999) (width 0.25) (layer F.Cu) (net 6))
 (segment (start 173.110002 113.615) (end 180.240001 120.744999) (width 0.25) (layer F.Cu) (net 6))
 (segment (start 182.150001 124.809999) (end 181.865 125.095) (width 0.25) (layer F.Cu) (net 6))
 (segment (start 172.725 113.615) (end 173.110002 113.615) (width 0.25) (layer F.Cu) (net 6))
 (segment (start 163.340001 114.440001) (end 162.565 113.665) (width 0.25) (layer F.Cu) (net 5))
 (segment (start 166.229999 114.440001) (end 163.340001 114.440001) (width 0.25) (layer F.Cu) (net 5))
 (segment (start 167.005 113.665) (end 166.229999 114.440001) (width 0.25) (layer F.Cu) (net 5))
 (segment (start 159.765 113.665) (end 162.565 113.665) (width 0.25) (layer F.Cu) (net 5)))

